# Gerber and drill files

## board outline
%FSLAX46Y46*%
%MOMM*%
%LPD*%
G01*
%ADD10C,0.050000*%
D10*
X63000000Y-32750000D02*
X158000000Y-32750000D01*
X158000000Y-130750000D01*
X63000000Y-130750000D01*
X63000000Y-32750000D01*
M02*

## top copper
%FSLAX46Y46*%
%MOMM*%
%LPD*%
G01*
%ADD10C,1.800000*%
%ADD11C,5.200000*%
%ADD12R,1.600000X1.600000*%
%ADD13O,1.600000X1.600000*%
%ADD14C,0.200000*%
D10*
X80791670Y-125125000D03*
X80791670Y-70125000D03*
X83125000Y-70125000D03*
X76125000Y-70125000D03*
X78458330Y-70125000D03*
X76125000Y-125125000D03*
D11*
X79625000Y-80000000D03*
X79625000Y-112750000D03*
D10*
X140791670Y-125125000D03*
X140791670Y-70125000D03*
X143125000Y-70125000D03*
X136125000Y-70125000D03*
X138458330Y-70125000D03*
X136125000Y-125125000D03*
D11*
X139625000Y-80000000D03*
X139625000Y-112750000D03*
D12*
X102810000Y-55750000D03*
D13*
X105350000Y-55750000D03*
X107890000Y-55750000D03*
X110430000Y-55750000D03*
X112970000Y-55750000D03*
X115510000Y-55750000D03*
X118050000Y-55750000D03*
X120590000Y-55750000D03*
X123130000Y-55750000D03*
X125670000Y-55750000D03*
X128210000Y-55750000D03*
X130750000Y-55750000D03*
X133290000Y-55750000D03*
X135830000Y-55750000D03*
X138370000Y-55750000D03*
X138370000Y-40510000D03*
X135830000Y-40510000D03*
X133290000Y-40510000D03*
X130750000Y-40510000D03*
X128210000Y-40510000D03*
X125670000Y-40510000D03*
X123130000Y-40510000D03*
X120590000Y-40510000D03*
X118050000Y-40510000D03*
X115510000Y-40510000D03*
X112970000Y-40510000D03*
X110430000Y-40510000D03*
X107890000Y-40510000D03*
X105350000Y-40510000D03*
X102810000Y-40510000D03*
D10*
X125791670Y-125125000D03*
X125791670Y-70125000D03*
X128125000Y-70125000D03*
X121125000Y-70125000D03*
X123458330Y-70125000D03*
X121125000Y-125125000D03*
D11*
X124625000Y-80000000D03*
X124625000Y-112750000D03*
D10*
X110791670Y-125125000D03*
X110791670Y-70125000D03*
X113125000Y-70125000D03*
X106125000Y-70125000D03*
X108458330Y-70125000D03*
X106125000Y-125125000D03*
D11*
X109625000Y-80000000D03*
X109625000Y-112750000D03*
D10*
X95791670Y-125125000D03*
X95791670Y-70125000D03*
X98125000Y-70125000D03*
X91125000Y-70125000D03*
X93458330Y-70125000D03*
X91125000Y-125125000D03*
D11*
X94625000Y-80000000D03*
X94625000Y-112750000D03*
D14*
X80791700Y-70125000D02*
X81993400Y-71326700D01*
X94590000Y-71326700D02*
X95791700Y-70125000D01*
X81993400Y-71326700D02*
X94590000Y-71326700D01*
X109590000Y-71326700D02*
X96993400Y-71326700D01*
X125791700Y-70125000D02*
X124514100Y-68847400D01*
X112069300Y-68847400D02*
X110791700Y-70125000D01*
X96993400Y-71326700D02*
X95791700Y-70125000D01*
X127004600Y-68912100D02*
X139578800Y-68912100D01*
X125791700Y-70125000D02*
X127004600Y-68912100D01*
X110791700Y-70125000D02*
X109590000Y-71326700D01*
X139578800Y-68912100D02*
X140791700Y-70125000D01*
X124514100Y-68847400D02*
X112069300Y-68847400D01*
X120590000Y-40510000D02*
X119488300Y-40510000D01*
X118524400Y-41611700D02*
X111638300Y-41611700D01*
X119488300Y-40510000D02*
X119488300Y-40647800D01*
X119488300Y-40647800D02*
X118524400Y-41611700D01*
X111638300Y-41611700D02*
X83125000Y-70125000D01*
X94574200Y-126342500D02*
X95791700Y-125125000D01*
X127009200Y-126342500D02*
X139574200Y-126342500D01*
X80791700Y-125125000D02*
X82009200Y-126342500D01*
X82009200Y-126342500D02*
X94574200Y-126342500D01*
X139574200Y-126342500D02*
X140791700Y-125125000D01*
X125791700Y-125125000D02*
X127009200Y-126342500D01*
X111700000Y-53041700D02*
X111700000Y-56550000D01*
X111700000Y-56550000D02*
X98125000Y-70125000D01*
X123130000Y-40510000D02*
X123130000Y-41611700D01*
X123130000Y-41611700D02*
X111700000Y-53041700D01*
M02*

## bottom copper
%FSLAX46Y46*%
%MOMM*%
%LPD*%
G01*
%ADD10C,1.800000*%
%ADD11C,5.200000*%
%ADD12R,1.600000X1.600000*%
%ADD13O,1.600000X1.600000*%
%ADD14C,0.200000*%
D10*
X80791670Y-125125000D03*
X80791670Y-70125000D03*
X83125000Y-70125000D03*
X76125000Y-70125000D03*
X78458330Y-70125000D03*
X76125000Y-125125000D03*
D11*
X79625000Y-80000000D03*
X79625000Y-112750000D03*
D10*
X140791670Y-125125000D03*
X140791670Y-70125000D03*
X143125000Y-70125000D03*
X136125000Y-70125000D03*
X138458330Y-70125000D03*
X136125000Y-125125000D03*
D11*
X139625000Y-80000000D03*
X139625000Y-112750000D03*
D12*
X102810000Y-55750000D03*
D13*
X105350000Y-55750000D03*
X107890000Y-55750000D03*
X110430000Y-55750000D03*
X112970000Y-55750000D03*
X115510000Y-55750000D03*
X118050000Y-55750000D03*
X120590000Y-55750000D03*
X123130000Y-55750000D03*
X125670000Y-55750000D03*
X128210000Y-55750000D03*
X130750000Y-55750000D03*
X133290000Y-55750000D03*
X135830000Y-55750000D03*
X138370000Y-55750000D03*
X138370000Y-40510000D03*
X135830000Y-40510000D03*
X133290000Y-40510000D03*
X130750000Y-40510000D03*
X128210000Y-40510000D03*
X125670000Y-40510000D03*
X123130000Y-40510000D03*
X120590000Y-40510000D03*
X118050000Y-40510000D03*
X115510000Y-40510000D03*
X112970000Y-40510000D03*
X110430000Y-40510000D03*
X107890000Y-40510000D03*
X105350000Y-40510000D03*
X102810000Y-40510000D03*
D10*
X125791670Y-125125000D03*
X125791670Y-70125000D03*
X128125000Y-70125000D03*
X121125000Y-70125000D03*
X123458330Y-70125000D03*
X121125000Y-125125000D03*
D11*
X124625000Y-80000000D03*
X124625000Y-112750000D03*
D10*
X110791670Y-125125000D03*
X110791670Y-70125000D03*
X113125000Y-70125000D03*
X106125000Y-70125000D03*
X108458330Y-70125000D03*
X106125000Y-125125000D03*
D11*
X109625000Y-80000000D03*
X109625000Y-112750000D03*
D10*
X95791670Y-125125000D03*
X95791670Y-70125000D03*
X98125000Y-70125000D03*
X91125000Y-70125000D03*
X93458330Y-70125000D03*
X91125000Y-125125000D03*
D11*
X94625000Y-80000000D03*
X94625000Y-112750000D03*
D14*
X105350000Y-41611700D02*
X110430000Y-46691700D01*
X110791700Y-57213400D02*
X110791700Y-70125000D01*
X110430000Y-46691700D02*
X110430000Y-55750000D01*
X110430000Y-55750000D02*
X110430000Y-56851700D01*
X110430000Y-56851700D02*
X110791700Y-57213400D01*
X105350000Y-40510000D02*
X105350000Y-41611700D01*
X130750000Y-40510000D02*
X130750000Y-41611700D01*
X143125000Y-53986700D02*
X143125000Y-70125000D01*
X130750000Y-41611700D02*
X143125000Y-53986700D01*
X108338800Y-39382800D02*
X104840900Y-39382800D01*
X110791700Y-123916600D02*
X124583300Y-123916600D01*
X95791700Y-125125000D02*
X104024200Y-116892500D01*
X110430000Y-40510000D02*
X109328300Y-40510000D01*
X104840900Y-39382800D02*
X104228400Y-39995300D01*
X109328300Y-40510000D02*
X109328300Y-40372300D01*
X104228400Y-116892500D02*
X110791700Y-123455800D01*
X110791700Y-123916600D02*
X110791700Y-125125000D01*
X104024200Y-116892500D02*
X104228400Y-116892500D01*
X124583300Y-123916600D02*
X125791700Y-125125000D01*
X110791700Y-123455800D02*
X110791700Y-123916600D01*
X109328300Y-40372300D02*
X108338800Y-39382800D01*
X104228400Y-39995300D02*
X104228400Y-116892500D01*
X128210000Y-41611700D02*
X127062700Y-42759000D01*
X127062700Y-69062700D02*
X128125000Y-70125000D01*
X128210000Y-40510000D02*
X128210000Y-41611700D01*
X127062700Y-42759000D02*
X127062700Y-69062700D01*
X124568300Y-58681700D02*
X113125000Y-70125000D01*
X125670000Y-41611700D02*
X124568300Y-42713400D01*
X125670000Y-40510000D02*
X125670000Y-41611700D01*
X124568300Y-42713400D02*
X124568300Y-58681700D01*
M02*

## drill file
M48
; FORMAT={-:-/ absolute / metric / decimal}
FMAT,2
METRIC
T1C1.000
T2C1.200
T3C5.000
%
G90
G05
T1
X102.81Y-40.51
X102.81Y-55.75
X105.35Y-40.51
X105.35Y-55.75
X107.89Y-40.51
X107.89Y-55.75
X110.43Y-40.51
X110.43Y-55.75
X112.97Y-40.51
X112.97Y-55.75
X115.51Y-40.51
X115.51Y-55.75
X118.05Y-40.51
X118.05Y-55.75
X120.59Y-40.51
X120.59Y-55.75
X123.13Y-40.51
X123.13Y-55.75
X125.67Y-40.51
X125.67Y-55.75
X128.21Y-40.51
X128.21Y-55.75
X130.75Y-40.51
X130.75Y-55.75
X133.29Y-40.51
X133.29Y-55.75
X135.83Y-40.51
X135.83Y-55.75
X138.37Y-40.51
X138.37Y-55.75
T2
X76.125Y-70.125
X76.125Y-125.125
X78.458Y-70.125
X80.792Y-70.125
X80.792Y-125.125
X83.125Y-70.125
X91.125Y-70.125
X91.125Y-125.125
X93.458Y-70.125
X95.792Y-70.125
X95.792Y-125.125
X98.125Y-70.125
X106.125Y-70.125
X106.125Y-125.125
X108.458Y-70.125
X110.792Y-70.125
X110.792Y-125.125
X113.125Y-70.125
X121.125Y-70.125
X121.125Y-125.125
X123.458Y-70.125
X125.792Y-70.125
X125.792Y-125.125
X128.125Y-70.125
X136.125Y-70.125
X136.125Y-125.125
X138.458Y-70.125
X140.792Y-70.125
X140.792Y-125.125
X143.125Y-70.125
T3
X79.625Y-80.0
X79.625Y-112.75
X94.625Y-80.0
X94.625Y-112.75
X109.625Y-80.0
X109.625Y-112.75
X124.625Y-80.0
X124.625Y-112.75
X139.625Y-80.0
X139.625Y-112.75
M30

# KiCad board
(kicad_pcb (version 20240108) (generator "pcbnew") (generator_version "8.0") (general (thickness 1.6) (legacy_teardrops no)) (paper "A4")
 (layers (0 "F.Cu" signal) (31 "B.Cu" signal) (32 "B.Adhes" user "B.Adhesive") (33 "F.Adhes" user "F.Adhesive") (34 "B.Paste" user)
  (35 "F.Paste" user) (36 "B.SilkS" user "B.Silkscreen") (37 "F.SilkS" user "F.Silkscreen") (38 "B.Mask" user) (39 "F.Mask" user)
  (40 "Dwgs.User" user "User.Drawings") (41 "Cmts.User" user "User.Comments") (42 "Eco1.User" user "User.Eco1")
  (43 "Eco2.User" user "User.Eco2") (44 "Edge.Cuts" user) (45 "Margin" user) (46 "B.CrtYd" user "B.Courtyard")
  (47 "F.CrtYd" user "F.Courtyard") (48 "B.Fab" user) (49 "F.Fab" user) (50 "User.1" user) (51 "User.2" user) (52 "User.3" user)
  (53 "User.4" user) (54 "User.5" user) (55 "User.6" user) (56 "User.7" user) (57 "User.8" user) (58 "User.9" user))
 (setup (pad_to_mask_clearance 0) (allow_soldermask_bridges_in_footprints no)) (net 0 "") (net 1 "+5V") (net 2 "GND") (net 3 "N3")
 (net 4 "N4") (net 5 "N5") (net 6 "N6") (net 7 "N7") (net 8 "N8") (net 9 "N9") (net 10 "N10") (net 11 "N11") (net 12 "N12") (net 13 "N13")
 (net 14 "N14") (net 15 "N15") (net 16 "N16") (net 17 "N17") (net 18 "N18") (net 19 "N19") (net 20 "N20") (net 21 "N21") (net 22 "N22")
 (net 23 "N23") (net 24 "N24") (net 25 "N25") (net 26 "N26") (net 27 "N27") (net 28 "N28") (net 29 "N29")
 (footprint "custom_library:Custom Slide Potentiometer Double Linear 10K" (layer "F.Cu") (at 75 67.5)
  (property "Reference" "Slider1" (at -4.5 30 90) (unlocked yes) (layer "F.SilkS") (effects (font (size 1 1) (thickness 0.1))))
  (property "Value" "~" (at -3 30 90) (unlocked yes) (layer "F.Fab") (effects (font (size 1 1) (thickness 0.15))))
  (pad "1" thru_hole circle (at 5.79167 57.625) (size 1.8 1.8) (drill 1.2) (layers "*.Cu" "*.Mask") (remove_unused_layers no) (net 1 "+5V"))
  (pad "2" thru_hole circle (at 5.79167 2.625) (size 1.8 1.8) (drill 1.2) (layers "*.Cu" "*.Mask") (remove_unused_layers no) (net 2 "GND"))
  (pad "3" thru_hole circle (at 8.125 2.625) (size 1.8 1.8) (drill 1.2) (layers "*.Cu" "*.Mask") (remove_unused_layers no) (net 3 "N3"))
  (pad "4" thru_hole circle (at 1.125 2.625) (size 1.8 1.8) (drill 1.2) (layers "*.Cu" "*.Mask") (remove_unused_layers no))
  (pad "5" thru_hole circle (at 3.45833 2.625) (size 1.8 1.8) (drill 1.2) (layers "*.Cu" "*.Mask") (remove_unused_layers no))
  (pad "6" thru_hole circle (at 1.125 57.625) (size 1.8 1.8) (drill 1.2) (layers "*.Cu" "*.Mask") (remove_unused_layers no))
  (pad "7" thru_hole circle (at 4.625 12.5) (size 5.2 5.2) (drill 5) (layers "*.Cu" "*.Mask") (remove_unused_layers no))
  (pad "8" thru_hole circle (at 4.625 45.25) (size 5.2 5.2) (drill 5) (layers "*.Cu" "*.Mask") (remove_unused_layers no)))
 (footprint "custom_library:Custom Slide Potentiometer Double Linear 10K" (layer "F.Cu") (at 135 67.5)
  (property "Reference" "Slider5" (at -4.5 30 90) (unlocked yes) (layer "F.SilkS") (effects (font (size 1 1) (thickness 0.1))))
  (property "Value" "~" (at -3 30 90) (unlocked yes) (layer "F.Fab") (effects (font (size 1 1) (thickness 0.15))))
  (pad "1" thru_hole circle (at 5.79167 57.625) (size 1.8 1.8) (drill 1.2) (layers "*.Cu" "*.Mask") (remove_unused_layers no) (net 1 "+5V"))
  (pad "2" thru_hole circle (at 5.79167 2.625) (size 1.8 1.8) (drill 1.2) (layers "*.Cu" "*.Mask") (remove_unused_layers no) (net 2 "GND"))
  (pad "3" thru_hole circle (at 8.125 2.625) (size 1.8 1.8) (drill 1.2) (layers "*.Cu" "*.Mask") (remove_unused_layers no) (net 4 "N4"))
  (pad "4" thru_hole circle (at 1.125 2.625) (size 1.8 1.8) (drill 1.2) (layers "*.Cu" "*.Mask") (remove_unused_layers no))
  (pad "5" thru_hole circle (at 3.45833 2.625) (size 1.8 1.8) (drill 1.2) (layers "*.Cu" "*.Mask") (remove_unused_layers no))
  (pad "6" thru_hole circle (at 1.125 57.625) (size 1.8 1.8) (drill 1.2) (layers "*.Cu" "*.Mask") (remove_unused_layers no))
  (pad "7" thru_hole circle (at 4.625 12.5) (size 5.2 5.2) (drill 5) (layers "*.Cu" "*.Mask") (remove_unused_layers no))
  (pad "8" thru_hole circle (at 4.625 45.25) (size 5.2 5.2) (drill 5) (layers "*.Cu" "*.Mask") (remove_unused_layers no)))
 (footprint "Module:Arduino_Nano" (layer "F.Cu") (at 102.81 55.75 90)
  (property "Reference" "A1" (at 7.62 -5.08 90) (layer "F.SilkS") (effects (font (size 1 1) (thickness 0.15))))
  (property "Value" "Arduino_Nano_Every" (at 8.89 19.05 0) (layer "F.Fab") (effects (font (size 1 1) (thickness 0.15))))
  (pad "1" thru_hole rect (at 0 0 90) (size 1.6 1.6) (drill 1) (layers "*.Cu" "*.Mask") (remove_unused_layers no) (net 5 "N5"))
  (pad "2" thru_hole oval (at 0 2.54 90) (size 1.6 1.6) (drill 1) (layers "*.Cu" "*.Mask") (remove_unused_layers no) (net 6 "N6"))
  (pad "3" thru_hole oval (at 0 5.08 90) (size 1.6 1.6) (drill 1) (layers "*.Cu" "*.Mask") (remove_unused_layers no) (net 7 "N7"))
  (pad "4" thru_hole oval (at 0 7.62 90) (size 1.6 1.6) (drill 1) (layers "*.Cu" "*.Mask") (remove_unused_layers no) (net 2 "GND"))
  (pad "5" thru_hole oval (at 0 10.16 90) (size 1.6 1.6) (drill 1) (layers "*.Cu" "*.Mask") (remove_unused_layers no) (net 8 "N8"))
  (pad "6" thru_hole oval (at 0 12.7 90) (size 1.6 1.6) (drill 1) (layers "*.Cu" "*.Mask") (remove_unused_layers no) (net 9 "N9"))
  (pad "7" thru_hole oval (at 0 15.24 90) (size 1.6 1.6) (drill 1) (layers "*.Cu" "*.Mask") (remove_unused_layers no) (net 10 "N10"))
  (pad "8" thru_hole oval (at 0 17.78 90) (size 1.6 1.6) (drill 1) (layers "*.Cu" "*.Mask") (remove_unused_layers no) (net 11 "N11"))
  (pad "9" thru_hole oval (at 0 20.32 90) (size 1.6 1.6) (drill 1) (layers "*.Cu" "*.Mask") (remove_unused_layers no) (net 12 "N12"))
  (pad "10" thru_hole oval (at 0 22.86 90) (size 1.6 1.6) (drill 1) (layers "*.Cu" "*.Mask") (remove_unused_layers no) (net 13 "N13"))
  (pad "11" thru_hole oval (at 0 25.4 90) (size 1.6 1.6) (drill 1) (layers "*.Cu" "*.Mask") (remove_unused_layers no) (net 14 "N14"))
  (pad "12" thru_hole oval (at 0 27.94 90) (size 1.6 1.6) (drill 1) (layers "*.Cu" "*.Mask") (remove_unused_layers no) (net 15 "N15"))
  (pad "13" thru_hole oval (at 0 30.48 90) (size 1.6 1.6) (drill 1) (layers "*.Cu" "*.Mask") (remove_unused_layers no) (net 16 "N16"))
  (pad "14" thru_hole oval (at 0 33.02 90) (size 1.6 1.6) (drill 1) (layers "*.Cu" "*.Mask") (remove_unused_layers no) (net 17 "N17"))
  (pad "15" thru_hole oval (at 0 35.56 90) (size 1.6 1.6) (drill 1) (layers "*.Cu" "*.Mask") (remove_unused_layers no) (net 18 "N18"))
  (pad "16" thru_hole oval (at 15.24 35.56 90) (size 1.6 1.6) (drill 1) (layers "*.Cu" "*.Mask") (remove_unused_layers no) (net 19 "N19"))
  (pad "17" thru_hole oval (at 15.24 33.02 90) (size 1.6 1.6) (drill 1) (layers "*.Cu" "*.Mask") (remove_unused_layers no) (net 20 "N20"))
  (pad "18" thru_hole oval (at 15.24 30.48 90) (size 1.6 1.6) (drill 1) (layers "*.Cu" "*.Mask") (remove_unused_layers no) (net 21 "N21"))
  (pad "19" thru_hole oval (at 15.24 27.94 90) (size 1.6 1.6) (drill 1) (layers "*.Cu" "*.Mask") (remove_unused_layers no) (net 4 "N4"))
  (pad "20" thru_hole oval (at 15.24 25.4 90) (size 1.6 1.6) (drill 1) (layers "*.Cu" "*.Mask") (remove_unused_layers no) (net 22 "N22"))
  (pad "21" thru_hole oval (at 15.24 22.86 90) (size 1.6 1.6) (drill 1) (layers "*.Cu" "*.Mask") (remove_unused_layers no) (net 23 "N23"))
  (pad "22" thru_hole oval (at 15.24 20.32 90) (size 1.6 1.6) (drill 1) (layers "*.Cu" "*.Mask") (remove_unused_layers no) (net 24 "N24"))
  (pad "23" thru_hole oval (at 15.24 17.78 90) (size 1.6 1.6) (drill 1) (layers "*.Cu" "*.Mask") (remove_unused_layers no) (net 3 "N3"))
  (pad "24" thru_hole oval (at 15.24 15.24 90) (size 1.6 1.6) (drill 1) (layers "*.Cu" "*.Mask") (remove_unused_layers no) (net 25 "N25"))
  (pad "25" thru_hole oval (at 15.24 12.7 90) (size 1.6 1.6) (drill 1) (layers "*.Cu" "*.Mask") (remove_unused_layers no) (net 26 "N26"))
  (pad "26" thru_hole oval (at 15.24 10.16 90) (size 1.6 1.6) (drill 1) (layers "*.Cu" "*.Mask") (remove_unused_layers no) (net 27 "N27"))
  (pad "27" thru_hole oval (at 15.24 7.62 90) (size 1.6 1.6) (drill 1) (layers "*.Cu" "*.Mask") (remove_unused_layers no) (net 1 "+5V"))
  (pad "28" thru_hole oval (at 15.24 5.08 90) (size 1.6 1.6) (drill 1) (layers "*.Cu" "*.Mask") (remove_unused_layers no) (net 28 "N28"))
  (pad "29" thru_hole oval (at 15.24 2.54 90) (size 1.6 1.6) (drill 1) (layers "*.Cu" "*.Mask") (remove_unused_layers no) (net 2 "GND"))
  (pad "30" thru_hole oval (at 15.24 0 90) (size 1.6 1.6) (drill 1) (layers "*.Cu" "*.Mask") (remove_unused_layers no) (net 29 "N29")))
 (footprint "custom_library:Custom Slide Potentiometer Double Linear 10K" (layer "F.Cu") (at 120 67.5)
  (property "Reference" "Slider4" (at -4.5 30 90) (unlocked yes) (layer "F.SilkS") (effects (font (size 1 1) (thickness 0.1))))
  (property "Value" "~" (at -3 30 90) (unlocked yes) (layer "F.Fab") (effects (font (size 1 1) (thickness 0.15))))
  (pad "1" thru_hole circle (at 5.79167 57.625) (size 1.8 1.8) (drill 1.2) (layers "*.Cu" "*.Mask") (remove_unused_layers no) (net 1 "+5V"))
  (pad "2" thru_hole circle (at 5.79167 2.625) (size 1.8 1.8) (drill 1.2) (layers "*.Cu" "*.Mask") (remove_unused_layers no) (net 2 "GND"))
  (pad "3" thru_hole circle (at 8.125 2.625) (size 1.8 1.8) (drill 1.2) (layers "*.Cu" "*.Mask") (remove_unused_layers no) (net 22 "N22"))
  (pad "4" thru_hole circle (at 1.125 2.625) (size 1.8 1.8) (drill 1.2) (layers "*.Cu" "*.Mask") (remove_unused_layers no))
  (pad "5" thru_hole circle (at 3.45833 2.625) (size 1.8 1.8) (drill 1.2) (layers "*.Cu" "*.Mask") (remove_unused_layers no))
  (pad "6" thru_hole circle (at 1.125 57.625) (size 1.8 1.8) (drill 1.2) (layers "*.Cu" "*.Mask") (remove_unused_layers no))
  (pad "7" thru_hole circle (at 4.625 12.5) (size 5.2 5.2) (drill 5) (layers "*.Cu" "*.Mask") (remove_unused_layers no))
  (pad "8" thru_hole circle (at 4.625 45.25) (size 5.2 5.2) (drill 5) (layers "*.Cu" "*.Mask") (remove_unused_layers no)))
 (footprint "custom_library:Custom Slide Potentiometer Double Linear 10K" (layer "F.Cu") (at 105 67.5)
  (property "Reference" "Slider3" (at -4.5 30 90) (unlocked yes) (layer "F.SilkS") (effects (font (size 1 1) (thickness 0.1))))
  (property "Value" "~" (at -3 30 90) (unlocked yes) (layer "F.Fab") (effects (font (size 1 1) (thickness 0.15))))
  (pad "1" thru_hole circle (at 5.79167 57.625) (size 1.8 1.8) (drill 1.2) (layers "*.Cu" "*.Mask") (remove_unused_layers no) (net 1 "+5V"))
  (pad "2" thru_hole circle (at 5.79167 2.625) (size 1.8 1.8) (drill 1.2) (layers "*.Cu" "*.Mask") (remove_unused_layers no) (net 2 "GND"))
  (pad "3" thru_hole circle (at 8.125 2.625) (size 1.8 1.8) (drill 1.2) (layers "*.Cu" "*.Mask") (remove_unused_layers no) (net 23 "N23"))
  (pad "4" thru_hole circle (at 1.125 2.625) (size 1.8 1.8) (drill 1.2) (layers "*.Cu" "*.Mask") (remove_unused_layers no))
  (pad "5" thru_hole circle (at 3.45833 2.625) (size 1.8 1.8) (drill 1.2) (layers "*.Cu" "*.Mask") (remove_unused_layers no))
  (pad "6" thru_hole circle (at 1.125 57.625) (size 1.8 1.8) (drill 1.2) (layers "*.Cu" "*.Mask") (remove_unused_layers no))
  (pad "7" thru_hole circle (at 4.625 12.5) (size 5.2 5.2) (drill 5) (layers "*.Cu" "*.Mask") (remove_unused_layers no))
  (pad "8" thru_hole circle (at 4.625 45.25) (size 5.2 5.2) (drill 5) (layers "*.Cu" "*.Mask") (remove_unused_layers no)))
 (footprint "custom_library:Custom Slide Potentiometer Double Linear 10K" (layer "F.Cu") (at 90 67.5)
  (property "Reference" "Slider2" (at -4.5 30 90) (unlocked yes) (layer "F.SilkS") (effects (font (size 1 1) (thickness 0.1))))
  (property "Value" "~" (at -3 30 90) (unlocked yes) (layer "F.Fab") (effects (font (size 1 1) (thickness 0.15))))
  (pad "1" thru_hole circle (at 5.79167 57.625) (size 1.8 1.8) (drill 1.2) (layers "*.Cu" "*.Mask") (remove_unused_layers no) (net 1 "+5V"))
  (pad "2" thru_hole circle (at 5.79167 2.625) (size 1.8 1.8) (drill 1.2) (layers "*.Cu" "*.Mask") (remove_unused_layers no) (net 2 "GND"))
  (pad "3" thru_hole circle (at 8.125 2.625) (size 1.8 1.8) (drill 1.2) (layers "*.Cu" "*.Mask") (remove_unused_layers no) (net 24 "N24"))
  (pad "4" thru_hole circle (at 1.125 2.625) (size 1.8 1.8) (drill 1.2) (layers "*.Cu" "*.Mask") (remove_unused_layers no))
  (pad "5" thru_hole circle (at 3.45833 2.625) (size 1.8 1.8) (drill 1.2) (layers "*.Cu" "*.Mask") (remove_unused_layers no))
  (pad "6" thru_hole circle (at 1.125 57.625) (size 1.8 1.8) (drill 1.2) (layers "*.Cu" "*.Mask") (remove_unused_layers no))
  (pad "7" thru_hole circle (at 4.625 12.5) (size 5.2 5.2) (drill 5) (layers "*.Cu" "*.Mask") (remove_unused_layers no))
  (pad "8" thru_hole circle (at 4.625 45.25) (size 5.2 5.2) (drill 5) (layers "*.Cu" "*.Mask") (remove_unused_layers no)))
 (gr_rect (start 63 32.75) (end 158 130.75) (stroke (width 0.05) (type default)) (fill none) (layer "Edge.Cuts"))
 (segment (start 80.7917 70.125) (end 81.9934 71.3267) (width 0.2) (layer "F.Cu") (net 2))
 (segment (start 94.59 71.3267) (end 95.7917 70.125) (width 0.2) (layer "F.Cu") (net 2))
 (segment (start 81.9934 71.3267) (end 94.59 71.3267) (width 0.2) (layer "F.Cu") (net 2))
 (segment (start 109.59 71.3267) (end 96.9934 71.3267) (width 0.2) (layer "F.Cu") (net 2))
 (segment (start 125.7917 70.125) (end 124.5141 68.8474) (width 0.2) (layer "F.Cu") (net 2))
 (segment (start 112.0693 68.8474) (end 110.7917 70.125) (width 0.2) (layer "F.Cu") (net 2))
 (segment (start 96.9934 71.3267) (end 95.7917 70.125) (width 0.2) (layer "F.Cu") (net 2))
 (segment (start 127.0046 68.9121) (end 139.5788 68.9121) (width 0.2) (layer "F.Cu") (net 2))
 (segment (start 125.7917 70.125) (end 127.0046 68.9121) (width 0.2) (layer "F.Cu") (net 2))
 (segment (start 110.7917 70.125) (end 109.59 71.3267) (width 0.2) (layer "F.Cu") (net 2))
 (segment (start 139.5788 68.9121) (end 140.7917 70.125) (width 0.2) (layer "F.Cu") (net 2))
 (segment (start 124.5141 68.8474) (end 112.0693 68.8474) (width 0.2) (layer "F.Cu") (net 2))
 (segment (start 105.35 41.6117) (end 110.43 46.6917) (width 0.2) (layer "B.Cu") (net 2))
 (segment (start 110.7917 57.2134) (end 110.7917 70.125) (width 0.2) (layer "B.Cu") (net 2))
 (segment (start 110.43 46.6917) (end 110.43 55.75) (width 0.2) (layer "B.Cu") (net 2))
 (segment (start 110.43 55.75) (end 110.43 56.8517) (width 0.2) (layer "B.Cu") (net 2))
 (segment (start 110.43 56.8517) (end 110.7917 57.2134) (width 0.2) (layer "B.Cu") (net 2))
 (segment (start 105.35 40.51) (end 105.35 41.6117) (width 0.2) (layer "B.Cu") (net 2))
 (segment (start 130.75 40.51) (end 130.75 41.6117) (width 0.2) (layer "B.Cu") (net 4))
 (segment (start 143.125 53.9867) (end 143.125 70.125) (width 0.2) (layer "B.Cu") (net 4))
 (segment (start 130.75 41.6117) (end 143.125 53.9867) (width 0.2) (layer "B.Cu") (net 4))
 (segment (start 120.59 40.51) (end 119.4883 40.51) (width 0.2) (layer "F.Cu") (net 3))
 (segment (start 118.5244 41.6117) (end 111.6383 41.6117) (width 0.2) (layer "F.Cu") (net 3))
 (segment (start 119.4883 40.51) (end 119.4883 40.6478) (width 0.2) (layer "F.Cu") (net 3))
 (segment (start 119.4883 40.6478) (end 118.5244 41.6117) (width 0.2) (layer "F.Cu") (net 3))
 (segment (start 111.6383 41.6117) (end 83.125 70.125) (width 0.2) (layer "F.Cu") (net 3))
 (segment (start 94.5742 126.3425) (end 95.7917 125.125) (width 0.2) (layer "F.Cu") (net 1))
 (segment (start 127.0092 126.3425) (end 139.5742 126.3425) (width 0.2) (layer "F.Cu") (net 1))
 (segment (start 80.7917 125.125) (end 82.0092 126.3425) (width 0.2) (layer "F.Cu") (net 1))
 (segment (start 82.0092 126.3425) (end 94.5742 126.3425) (width 0.2) (layer "F.Cu") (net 1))
 (segment (start 139.5742 126.3425) (end 140.7917 125.125) (width 0.2) (layer "F.Cu") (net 1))
 (segment (start 125.7917 125.125) (end 127.0092 126.3425) (width 0.2) (layer "F.Cu") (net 1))
 (segment (start 108.3388 39.3828) (end 104.8409 39.3828) (width 0.2) (layer "B.Cu") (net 1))
 (segment (start 110.7917 123.9166) (end 124.5833 123.9166) (width 0.2) (layer "B.Cu") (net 1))
 (segment (start 95.7917 125.125) (end 104.0242 116.8925) (width 0.2) (layer "B.Cu") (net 1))
 (segment (start 110.43 40.51) (end 109.3283 40.51) (width 0.2) (layer "B.Cu") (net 1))
 (segment (start 104.8409 39.3828) (end 104.2284 39.9953) (width 0.2) (layer "B.Cu") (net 1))
 (segment (start 109.3283 40.51) (end 109.3283 40.3723) (width 0.2) (layer "B.Cu") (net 1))
 (segment (start 104.2284 116.8925) (end 110.7917 123.4558) (width 0.2) (layer "B.Cu") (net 1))
 (segment (start 110.7917 123.9166) (end 110.7917 125.125) (width 0.2) (layer "B.Cu") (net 1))
 (segment (start 104.0242 116.8925) (end 104.2284 116.8925) (width 0.2) (layer "B.Cu") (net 1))
 (segment (start 124.5833 123.9166) (end 125.7917 125.125) (width 0.2) (layer "B.Cu") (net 1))
 (segment (start 110.7917 123.4558) (end 110.7917 123.9166) (width 0.2) (layer "B.Cu") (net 1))
 (segment (start 109.3283 40.3723) (end 108.3388 39.3828) (width 0.2) (layer "B.Cu") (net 1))
 (segment (start 104.2284 39.9953) (end 104.2284 116.8925) (width 0.2) (layer "B.Cu") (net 1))
 (segment (start 111.7 53.0417) (end 111.7 56.55) (width 0.2) (layer "F.Cu") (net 24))
 (segment (start 111.7 56.55) (end 98.125 70.125) (width 0.2) (layer "F.Cu") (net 24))
 (segment (start 123.13 40.51) (end 123.13 41.6117) (width 0.2) (layer "F.Cu") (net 24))
 (segment (start 123.13 41.6117) (end 111.7 53.0417) (width 0.2) (layer "F.Cu") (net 24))
 (segment (start 128.21 41.6117) (end 127.0627 42.759) (width 0.2) (layer "B.Cu") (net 22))
 (segment (start 127.0627 69.0627) (end 128.125 70.125) (width 0.2) (layer "B.Cu") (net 22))
 (segment (start 128.21 40.51) (end 128.21 41.6117) (width 0.2) (layer "B.Cu") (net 22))
 (segment (start 127.0627 42.759) (end 127.0627 69.0627) (width 0.2) (layer "B.Cu") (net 22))
 (segment (start 124.5683 58.6817) (end 113.125 70.125) (width 0.2) (layer "B.Cu") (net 23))
 (segment (start 125.67 41.6117) (end 124.5683 42.7134) (width 0.2) (layer "B.Cu") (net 23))
 (segment (start 125.67 40.51) (end 125.67 41.6117) (width 0.2) (layer "B.Cu") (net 23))
 (segment (start 124.5683 42.7134) (end 124.5683 58.6817) (width 0.2) (layer "B.Cu") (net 23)))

